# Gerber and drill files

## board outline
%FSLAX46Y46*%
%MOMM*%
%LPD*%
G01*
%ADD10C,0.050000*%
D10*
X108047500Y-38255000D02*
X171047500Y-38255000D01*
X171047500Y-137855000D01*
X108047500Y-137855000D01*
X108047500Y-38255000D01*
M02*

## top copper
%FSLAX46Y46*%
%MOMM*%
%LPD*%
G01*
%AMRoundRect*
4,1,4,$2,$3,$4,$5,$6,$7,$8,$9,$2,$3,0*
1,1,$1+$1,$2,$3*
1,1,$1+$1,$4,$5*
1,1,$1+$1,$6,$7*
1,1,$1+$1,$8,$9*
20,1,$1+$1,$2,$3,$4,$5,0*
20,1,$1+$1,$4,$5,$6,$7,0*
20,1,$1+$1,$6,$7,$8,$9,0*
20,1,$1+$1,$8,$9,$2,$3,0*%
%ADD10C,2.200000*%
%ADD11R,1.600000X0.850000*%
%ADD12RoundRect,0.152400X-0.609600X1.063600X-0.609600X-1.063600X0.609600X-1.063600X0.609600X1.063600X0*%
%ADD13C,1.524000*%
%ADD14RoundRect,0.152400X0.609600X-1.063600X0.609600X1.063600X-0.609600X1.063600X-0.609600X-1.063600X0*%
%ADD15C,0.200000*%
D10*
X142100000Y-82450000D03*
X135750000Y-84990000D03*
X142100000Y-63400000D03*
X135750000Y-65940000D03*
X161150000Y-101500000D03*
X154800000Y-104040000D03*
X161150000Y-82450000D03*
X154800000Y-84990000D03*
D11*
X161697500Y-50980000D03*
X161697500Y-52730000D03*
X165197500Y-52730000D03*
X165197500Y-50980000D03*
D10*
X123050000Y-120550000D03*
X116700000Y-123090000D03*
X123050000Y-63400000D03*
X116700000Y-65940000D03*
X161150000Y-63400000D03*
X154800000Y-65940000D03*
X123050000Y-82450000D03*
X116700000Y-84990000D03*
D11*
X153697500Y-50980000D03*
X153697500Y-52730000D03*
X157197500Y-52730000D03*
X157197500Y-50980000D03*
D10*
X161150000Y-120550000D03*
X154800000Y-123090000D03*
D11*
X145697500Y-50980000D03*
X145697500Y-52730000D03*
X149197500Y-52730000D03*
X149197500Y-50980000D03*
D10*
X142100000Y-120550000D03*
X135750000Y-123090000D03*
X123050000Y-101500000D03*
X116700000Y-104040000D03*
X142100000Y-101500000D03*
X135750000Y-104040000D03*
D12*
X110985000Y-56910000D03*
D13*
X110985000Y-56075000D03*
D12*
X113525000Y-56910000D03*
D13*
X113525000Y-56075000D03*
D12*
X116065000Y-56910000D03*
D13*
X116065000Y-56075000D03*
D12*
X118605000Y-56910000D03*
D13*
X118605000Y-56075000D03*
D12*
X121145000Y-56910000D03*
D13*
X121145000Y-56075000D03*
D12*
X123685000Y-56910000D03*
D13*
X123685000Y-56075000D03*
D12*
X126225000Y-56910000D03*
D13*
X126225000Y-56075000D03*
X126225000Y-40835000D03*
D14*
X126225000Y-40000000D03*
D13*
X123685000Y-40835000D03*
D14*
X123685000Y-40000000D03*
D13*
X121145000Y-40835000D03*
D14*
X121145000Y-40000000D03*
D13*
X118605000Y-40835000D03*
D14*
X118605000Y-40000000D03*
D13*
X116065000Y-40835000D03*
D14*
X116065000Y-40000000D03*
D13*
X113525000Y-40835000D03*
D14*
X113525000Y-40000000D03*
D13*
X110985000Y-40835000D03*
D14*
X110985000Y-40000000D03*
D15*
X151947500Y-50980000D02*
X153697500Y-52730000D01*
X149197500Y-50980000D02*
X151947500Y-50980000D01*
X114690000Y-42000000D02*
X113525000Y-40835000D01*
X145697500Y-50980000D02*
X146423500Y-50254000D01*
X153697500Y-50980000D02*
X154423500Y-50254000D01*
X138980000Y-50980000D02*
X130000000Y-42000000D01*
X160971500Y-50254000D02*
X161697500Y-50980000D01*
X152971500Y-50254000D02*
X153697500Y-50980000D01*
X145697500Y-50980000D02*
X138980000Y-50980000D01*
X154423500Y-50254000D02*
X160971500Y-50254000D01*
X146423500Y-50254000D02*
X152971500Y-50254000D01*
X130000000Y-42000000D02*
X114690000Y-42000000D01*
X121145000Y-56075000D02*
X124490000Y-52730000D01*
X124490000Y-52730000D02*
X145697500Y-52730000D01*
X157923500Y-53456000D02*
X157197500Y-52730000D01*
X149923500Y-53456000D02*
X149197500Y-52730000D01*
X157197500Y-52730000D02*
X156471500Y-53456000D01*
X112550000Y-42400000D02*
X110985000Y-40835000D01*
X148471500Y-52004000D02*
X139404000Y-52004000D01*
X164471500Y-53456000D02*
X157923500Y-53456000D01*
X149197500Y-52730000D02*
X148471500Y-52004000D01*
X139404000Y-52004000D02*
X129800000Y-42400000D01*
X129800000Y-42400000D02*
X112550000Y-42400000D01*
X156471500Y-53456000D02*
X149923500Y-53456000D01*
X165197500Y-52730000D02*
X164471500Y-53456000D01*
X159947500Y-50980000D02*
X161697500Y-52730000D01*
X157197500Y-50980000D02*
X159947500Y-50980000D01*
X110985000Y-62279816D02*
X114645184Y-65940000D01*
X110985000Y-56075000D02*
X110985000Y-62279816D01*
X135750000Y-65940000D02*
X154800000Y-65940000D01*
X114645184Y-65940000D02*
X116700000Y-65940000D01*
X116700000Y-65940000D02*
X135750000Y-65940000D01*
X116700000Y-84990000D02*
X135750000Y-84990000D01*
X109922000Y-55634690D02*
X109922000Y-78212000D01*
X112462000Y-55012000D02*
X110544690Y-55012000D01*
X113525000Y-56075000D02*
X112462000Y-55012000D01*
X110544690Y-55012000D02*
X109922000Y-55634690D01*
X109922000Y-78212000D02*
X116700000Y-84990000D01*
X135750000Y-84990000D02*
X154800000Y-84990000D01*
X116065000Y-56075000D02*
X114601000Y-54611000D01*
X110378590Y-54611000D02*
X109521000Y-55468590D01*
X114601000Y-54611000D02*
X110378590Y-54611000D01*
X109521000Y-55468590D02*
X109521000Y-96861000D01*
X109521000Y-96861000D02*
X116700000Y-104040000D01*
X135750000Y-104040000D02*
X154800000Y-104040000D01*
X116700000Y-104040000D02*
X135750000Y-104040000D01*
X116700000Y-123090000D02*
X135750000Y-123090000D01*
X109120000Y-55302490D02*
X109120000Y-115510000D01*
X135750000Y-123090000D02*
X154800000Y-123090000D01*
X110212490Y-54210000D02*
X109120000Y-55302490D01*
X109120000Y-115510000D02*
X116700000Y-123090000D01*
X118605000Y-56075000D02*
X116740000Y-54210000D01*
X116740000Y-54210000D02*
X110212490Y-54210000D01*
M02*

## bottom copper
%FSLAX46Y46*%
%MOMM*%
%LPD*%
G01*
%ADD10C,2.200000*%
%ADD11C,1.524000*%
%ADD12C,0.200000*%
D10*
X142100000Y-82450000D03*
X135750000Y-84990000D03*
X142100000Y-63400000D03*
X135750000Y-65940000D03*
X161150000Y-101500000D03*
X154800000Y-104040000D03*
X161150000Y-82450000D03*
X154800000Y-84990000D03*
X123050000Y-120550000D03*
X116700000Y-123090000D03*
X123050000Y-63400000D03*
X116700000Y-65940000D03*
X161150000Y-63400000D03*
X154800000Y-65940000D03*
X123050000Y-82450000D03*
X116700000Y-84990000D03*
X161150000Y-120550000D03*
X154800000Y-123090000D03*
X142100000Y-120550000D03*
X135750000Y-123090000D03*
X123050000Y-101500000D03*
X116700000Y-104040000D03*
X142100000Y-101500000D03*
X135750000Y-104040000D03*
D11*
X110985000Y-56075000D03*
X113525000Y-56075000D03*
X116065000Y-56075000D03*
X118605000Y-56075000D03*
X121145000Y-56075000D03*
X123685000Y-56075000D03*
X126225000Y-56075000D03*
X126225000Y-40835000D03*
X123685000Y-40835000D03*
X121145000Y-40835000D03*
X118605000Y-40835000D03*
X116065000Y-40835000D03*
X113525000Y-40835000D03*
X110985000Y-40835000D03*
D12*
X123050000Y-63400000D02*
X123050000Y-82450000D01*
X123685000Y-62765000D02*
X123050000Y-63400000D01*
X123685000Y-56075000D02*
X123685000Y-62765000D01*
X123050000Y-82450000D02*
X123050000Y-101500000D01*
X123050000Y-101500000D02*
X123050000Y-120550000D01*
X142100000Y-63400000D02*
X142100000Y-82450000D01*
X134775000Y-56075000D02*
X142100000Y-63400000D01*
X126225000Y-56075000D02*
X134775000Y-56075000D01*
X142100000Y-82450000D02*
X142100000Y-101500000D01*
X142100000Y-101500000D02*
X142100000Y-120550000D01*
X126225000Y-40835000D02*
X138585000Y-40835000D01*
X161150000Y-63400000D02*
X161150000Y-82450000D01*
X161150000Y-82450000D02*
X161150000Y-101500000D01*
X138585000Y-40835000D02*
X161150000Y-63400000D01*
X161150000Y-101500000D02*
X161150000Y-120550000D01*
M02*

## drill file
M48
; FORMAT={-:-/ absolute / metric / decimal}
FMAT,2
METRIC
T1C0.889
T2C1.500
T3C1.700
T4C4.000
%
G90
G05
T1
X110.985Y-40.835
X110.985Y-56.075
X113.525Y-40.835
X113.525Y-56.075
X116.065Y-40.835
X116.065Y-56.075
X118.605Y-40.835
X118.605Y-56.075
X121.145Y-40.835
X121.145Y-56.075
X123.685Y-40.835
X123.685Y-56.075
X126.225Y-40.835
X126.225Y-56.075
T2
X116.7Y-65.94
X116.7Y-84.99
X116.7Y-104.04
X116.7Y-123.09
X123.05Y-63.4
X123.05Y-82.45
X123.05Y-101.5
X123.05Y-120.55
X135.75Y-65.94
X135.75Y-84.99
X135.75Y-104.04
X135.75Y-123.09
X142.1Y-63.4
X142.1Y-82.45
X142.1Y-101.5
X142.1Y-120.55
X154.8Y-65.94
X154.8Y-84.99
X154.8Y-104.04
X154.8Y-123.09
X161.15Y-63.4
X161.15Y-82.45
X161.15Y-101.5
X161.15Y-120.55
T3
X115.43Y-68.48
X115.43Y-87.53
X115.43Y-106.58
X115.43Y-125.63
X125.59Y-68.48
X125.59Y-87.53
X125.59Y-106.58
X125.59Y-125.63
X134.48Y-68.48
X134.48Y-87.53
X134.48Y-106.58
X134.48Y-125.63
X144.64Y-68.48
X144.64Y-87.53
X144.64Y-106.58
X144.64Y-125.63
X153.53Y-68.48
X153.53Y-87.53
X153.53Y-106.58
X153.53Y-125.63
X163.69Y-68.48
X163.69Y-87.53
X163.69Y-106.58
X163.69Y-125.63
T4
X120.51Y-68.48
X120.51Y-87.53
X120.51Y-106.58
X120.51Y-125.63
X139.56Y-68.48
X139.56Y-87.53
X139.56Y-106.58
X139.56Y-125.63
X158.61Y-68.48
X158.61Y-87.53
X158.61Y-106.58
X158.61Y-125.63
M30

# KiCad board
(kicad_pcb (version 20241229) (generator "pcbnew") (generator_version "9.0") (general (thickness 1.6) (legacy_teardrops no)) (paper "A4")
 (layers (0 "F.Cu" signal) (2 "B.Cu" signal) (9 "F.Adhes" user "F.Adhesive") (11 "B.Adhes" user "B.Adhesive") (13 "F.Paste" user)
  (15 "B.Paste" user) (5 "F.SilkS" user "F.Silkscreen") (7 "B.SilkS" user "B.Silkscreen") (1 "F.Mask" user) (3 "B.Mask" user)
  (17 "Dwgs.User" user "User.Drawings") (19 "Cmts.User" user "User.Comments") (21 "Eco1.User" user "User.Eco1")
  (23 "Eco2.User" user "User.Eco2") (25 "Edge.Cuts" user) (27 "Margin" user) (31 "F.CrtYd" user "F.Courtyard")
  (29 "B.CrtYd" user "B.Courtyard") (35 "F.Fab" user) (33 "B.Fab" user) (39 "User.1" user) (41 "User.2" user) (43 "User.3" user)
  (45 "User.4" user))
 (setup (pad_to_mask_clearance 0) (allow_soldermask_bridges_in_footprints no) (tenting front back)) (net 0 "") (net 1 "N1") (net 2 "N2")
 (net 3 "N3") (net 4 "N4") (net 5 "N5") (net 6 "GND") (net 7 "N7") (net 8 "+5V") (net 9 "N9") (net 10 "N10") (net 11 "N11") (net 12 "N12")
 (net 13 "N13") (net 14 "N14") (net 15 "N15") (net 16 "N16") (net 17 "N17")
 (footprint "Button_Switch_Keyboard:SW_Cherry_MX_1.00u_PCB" (layer "F.Cu") (at 142.1 82.45)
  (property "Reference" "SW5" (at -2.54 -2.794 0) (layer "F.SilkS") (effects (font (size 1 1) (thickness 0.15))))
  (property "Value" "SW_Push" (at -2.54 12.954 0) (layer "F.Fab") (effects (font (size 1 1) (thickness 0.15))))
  (pad "" np_thru_hole circle (at -7.62 5.08) (size 1.7 1.7) (drill 1.7) (layers "*.Cu" "*.Mask"))
  (pad "" np_thru_hole circle (at -2.54 5.08) (size 4 4) (drill 4) (layers "*.Cu" "*.Mask"))
  (pad "" np_thru_hole circle (at 2.54 5.08) (size 1.7 1.7) (drill 1.7) (layers "*.Cu" "*.Mask"))
  (pad "1" thru_hole circle (at 0 0) (size 2.2 2.2) (drill 1.5) (layers "*.Cu" "*.Mask") (remove_unused_layers no) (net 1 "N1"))
  (pad "2" thru_hole circle (at -6.35 2.54) (size 2.2 2.2) (drill 1.5) (layers "*.Cu" "*.Mask") (remove_unused_layers no) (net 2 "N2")))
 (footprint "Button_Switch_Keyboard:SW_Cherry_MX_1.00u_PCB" (layer "F.Cu") (at 142.1 63.4)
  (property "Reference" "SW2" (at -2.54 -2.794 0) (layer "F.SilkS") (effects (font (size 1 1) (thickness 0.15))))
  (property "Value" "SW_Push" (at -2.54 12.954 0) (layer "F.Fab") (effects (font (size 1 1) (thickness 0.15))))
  (pad "" np_thru_hole circle (at -7.62 5.08) (size 1.7 1.7) (drill 1.7) (layers "*.Cu" "*.Mask"))
  (pad "" np_thru_hole circle (at -2.54 5.08) (size 4 4) (drill 4) (layers "*.Cu" "*.Mask"))
  (pad "" np_thru_hole circle (at 2.54 5.08) (size 1.7 1.7) (drill 1.7) (layers "*.Cu" "*.Mask"))
  (pad "1" thru_hole circle (at 0 0) (size 2.2 2.2) (drill 1.5) (layers "*.Cu" "*.Mask") (remove_unused_layers no) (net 1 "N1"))
  (pad "2" thru_hole circle (at -6.35 2.54) (size 2.2 2.2) (drill 1.5) (layers "*.Cu" "*.Mask") (remove_unused_layers no) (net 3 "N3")))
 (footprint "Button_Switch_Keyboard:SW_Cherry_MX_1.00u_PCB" (layer "F.Cu") (at 161.15 101.5)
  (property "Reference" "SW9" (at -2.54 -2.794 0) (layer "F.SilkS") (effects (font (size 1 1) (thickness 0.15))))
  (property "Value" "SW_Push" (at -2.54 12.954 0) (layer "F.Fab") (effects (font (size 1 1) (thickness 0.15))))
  (pad "" np_thru_hole circle (at -7.62 5.08) (size 1.7 1.7) (drill 1.7) (layers "*.Cu" "*.Mask"))
  (pad "" np_thru_hole circle (at -2.54 5.08) (size 4 4) (drill 4) (layers "*.Cu" "*.Mask"))
  (pad "" np_thru_hole circle (at 2.54 5.08) (size 1.7 1.7) (drill 1.7) (layers "*.Cu" "*.Mask"))
  (pad "1" thru_hole circle (at 0 0) (size 2.2 2.2) (drill 1.5) (layers "*.Cu" "*.Mask") (remove_unused_layers no) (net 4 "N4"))
  (pad "2" thru_hole circle (at -6.35 2.54) (size 2.2 2.2) (drill 1.5) (layers "*.Cu" "*.Mask") (remove_unused_layers no) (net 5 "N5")))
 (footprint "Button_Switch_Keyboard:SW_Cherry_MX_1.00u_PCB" (layer "F.Cu") (at 161.15 82.45)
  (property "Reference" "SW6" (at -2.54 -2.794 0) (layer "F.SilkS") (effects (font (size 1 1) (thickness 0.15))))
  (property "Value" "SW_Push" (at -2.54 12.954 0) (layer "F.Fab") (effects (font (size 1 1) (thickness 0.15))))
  (pad "" np_thru_hole circle (at -7.62 5.08) (size 1.7 1.7) (drill 1.7) (layers "*.Cu" "*.Mask"))
  (pad "" np_thru_hole circle (at -2.54 5.08) (size 4 4) (drill 4) (layers "*.Cu" "*.Mask"))
  (pad "" np_thru_hole circle (at 2.54 5.08) (size 1.7 1.7) (drill 1.7) (layers "*.Cu" "*.Mask"))
  (pad "1" thru_hole circle (at 0 0) (size 2.2 2.2) (drill 1.5) (layers "*.Cu" "*.Mask") (remove_unused_layers no) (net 4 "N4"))
  (pad "2" thru_hole circle (at -6.35 2.54) (size 2.2 2.2) (drill 1.5) (layers "*.Cu" "*.Mask") (remove_unused_layers no) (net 2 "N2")))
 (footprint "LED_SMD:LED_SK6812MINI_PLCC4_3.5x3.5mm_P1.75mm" (layer "F.Cu") (at 163.4475 51.855)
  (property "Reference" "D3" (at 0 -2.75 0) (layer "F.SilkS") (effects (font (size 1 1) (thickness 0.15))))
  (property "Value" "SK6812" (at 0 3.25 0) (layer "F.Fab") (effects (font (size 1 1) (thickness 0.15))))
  (pad "1" smd rect (at -1.75 -0.875) (size 1.6 0.85) (layers "F.Cu" "F.Mask" "F.Paste") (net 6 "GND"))
  (pad "2" smd rect (at -1.75 0.875) (size 1.6 0.85) (layers "F.Cu" "F.Mask" "F.Paste") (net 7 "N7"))
  (pad "3" smd rect (at 1.75 0.875) (size 1.6 0.85) (layers "F.Cu" "F.Mask" "F.Paste") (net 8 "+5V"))
  (pad "4" smd rect (at 1.75 -0.875) (size 1.6 0.85) (layers "F.Cu" "F.Mask" "F.Paste") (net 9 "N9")))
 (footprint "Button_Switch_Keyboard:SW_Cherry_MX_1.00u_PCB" (layer "F.Cu") (at 123.05 120.55)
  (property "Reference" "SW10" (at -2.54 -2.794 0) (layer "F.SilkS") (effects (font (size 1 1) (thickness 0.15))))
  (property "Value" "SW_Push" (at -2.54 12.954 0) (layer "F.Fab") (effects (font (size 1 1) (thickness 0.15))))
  (pad "" np_thru_hole circle (at -7.62 5.08) (size 1.7 1.7) (drill 1.7) (layers "*.Cu" "*.Mask"))
  (pad "" np_thru_hole circle (at -2.54 5.08) (size 4 4) (drill 4) (layers "*.Cu" "*.Mask"))
  (pad "" np_thru_hole circle (at 2.54 5.08) (size 1.7 1.7) (drill 1.7) (layers "*.Cu" "*.Mask"))
  (pad "1" thru_hole circle (at 0 0) (size 2.2 2.2) (drill 1.5) (layers "*.Cu" "*.Mask") (remove_unused_layers no) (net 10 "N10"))
  (pad "2" thru_hole circle (at -6.35 2.54) (size 2.2 2.2) (drill 1.5) (layers "*.Cu" "*.Mask") (remove_unused_layers no) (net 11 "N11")))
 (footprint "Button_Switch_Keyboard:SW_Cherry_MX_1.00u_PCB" (layer "F.Cu") (at 123.05 63.4)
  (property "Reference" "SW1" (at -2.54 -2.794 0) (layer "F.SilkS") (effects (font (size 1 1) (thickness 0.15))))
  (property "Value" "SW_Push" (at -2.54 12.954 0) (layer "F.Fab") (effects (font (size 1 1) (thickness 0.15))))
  (pad "" np_thru_hole circle (at -7.62 5.08) (size 1.7 1.7) (drill 1.7) (layers "*.Cu" "*.Mask"))
  (pad "" np_thru_hole circle (at -2.54 5.08) (size 4 4) (drill 4) (layers "*.Cu" "*.Mask"))
  (pad "" np_thru_hole circle (at 2.54 5.08) (size 1.7 1.7) (drill 1.7) (layers "*.Cu" "*.Mask"))
  (pad "1" thru_hole circle (at 0 0) (size 2.2 2.2) (drill 1.5) (layers "*.Cu" "*.Mask") (remove_unused_layers no) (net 10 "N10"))
  (pad "2" thru_hole circle (at -6.35 2.54) (size 2.2 2.2) (drill 1.5) (layers "*.Cu" "*.Mask") (remove_unused_layers no) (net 3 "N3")))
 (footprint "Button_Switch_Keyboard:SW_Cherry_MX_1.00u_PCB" (layer "F.Cu") (at 161.15 63.4)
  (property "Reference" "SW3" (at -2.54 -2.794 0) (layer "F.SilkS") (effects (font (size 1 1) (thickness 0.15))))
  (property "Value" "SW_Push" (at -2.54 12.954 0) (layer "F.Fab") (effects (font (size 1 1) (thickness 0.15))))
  (pad "" np_thru_hole circle (at -7.62 5.08) (size 1.7 1.7) (drill 1.7) (layers "*.Cu" "*.Mask"))
  (pad "" np_thru_hole circle (at -2.54 5.08) (size 4 4) (drill 4) (layers "*.Cu" "*.Mask"))
  (pad "" np_thru_hole circle (at 2.54 5.08) (size 1.7 1.7) (drill 1.7) (layers "*.Cu" "*.Mask"))
  (pad "1" thru_hole circle (at 0 0) (size 2.2 2.2) (drill 1.5) (layers "*.Cu" "*.Mask") (remove_unused_layers no) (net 4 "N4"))
  (pad "2" thru_hole circle (at -6.35 2.54) (size 2.2 2.2) (drill 1.5) (layers "*.Cu" "*.Mask") (remove_unused_layers no) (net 3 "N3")))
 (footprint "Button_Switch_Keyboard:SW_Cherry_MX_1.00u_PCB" (layer "F.Cu") (at 123.05 82.45)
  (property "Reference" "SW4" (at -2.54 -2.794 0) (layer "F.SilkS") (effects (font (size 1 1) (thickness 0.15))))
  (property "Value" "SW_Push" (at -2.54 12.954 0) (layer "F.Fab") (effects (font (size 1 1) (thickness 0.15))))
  (pad "" np_thru_hole circle (at -7.62 5.08) (size 1.7 1.7) (drill 1.7) (layers "*.Cu" "*.Mask"))
  (pad "" np_thru_hole circle (at -2.54 5.08) (size 4 4) (drill 4) (layers "*.Cu" "*.Mask"))
  (pad "" np_thru_hole circle (at 2.54 5.08) (size 1.7 1.7) (drill 1.7) (layers "*.Cu" "*.Mask"))
  (pad "1" thru_hole circle (at 0 0) (size 2.2 2.2) (drill 1.5) (layers "*.Cu" "*.Mask") (remove_unused_layers no) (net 10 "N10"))
  (pad "2" thru_hole circle (at -6.35 2.54) (size 2.2 2.2) (drill 1.5) (layers "*.Cu" "*.Mask") (remove_unused_layers no) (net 2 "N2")))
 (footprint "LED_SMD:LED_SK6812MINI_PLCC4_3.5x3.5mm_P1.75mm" (layer "F.Cu") (at 155.4475 51.855)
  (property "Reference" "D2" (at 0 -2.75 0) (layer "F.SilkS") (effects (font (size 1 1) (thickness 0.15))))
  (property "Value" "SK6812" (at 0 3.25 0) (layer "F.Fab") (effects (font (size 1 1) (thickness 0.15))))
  (pad "1" smd rect (at -1.75 -0.875) (size 1.6 0.85) (layers "F.Cu" "F.Mask" "F.Paste") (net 6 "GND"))
  (pad "2" smd rect (at -1.75 0.875) (size 1.6 0.85) (layers "F.Cu" "F.Mask" "F.Paste") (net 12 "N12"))
  (pad "3" smd rect (at 1.75 0.875) (size 1.6 0.85) (layers "F.Cu" "F.Mask" "F.Paste") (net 8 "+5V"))
  (pad "4" smd rect (at 1.75 -0.875) (size 1.6 0.85) (layers "F.Cu" "F.Mask" "F.Paste") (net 7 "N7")))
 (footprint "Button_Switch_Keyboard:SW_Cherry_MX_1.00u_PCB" (layer "F.Cu") (at 161.15 120.55)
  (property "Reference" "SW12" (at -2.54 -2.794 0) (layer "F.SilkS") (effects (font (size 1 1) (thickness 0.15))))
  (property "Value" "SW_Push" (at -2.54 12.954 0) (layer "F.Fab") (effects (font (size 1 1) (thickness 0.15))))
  (pad "" np_thru_hole circle (at -7.62 5.08) (size 1.7 1.7) (drill 1.7) (layers "*.Cu" "*.Mask"))
  (pad "" np_thru_hole circle (at -2.54 5.08) (size 4 4) (drill 4) (layers "*.Cu" "*.Mask"))
  (pad "" np_thru_hole circle (at 2.54 5.08) (size 1.7 1.7) (drill 1.7) (layers "*.Cu" "*.Mask"))
  (pad "1" thru_hole circle (at 0 0) (size 2.2 2.2) (drill 1.5) (layers "*.Cu" "*.Mask") (remove_unused_layers no) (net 4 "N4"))
  (pad "2" thru_hole circle (at -6.35 2.54) (size 2.2 2.2) (drill 1.5) (layers "*.Cu" "*.Mask") (remove_unused_layers no) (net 11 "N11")))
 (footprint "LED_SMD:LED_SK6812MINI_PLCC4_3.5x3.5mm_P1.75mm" (layer "F.Cu") (at 147.4475 51.855)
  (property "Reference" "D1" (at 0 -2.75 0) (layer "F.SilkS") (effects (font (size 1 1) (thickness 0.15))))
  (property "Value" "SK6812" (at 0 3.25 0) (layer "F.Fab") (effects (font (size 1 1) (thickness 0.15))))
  (pad "1" smd rect (at -1.75 -0.875) (size 1.6 0.85) (layers "F.Cu" "F.Mask" "F.Paste") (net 6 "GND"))
  (pad "2" smd rect (at -1.75 0.875) (size 1.6 0.85) (layers "F.Cu" "F.Mask" "F.Paste") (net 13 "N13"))
  (pad "3" smd rect (at 1.75 0.875) (size 1.6 0.85) (layers "F.Cu" "F.Mask" "F.Paste") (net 8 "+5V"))
  (pad "4" smd rect (at 1.75 -0.875) (size 1.6 0.85) (layers "F.Cu" "F.Mask" "F.Paste") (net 12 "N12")))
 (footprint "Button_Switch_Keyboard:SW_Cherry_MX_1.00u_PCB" (layer "F.Cu") (at 142.1 120.55)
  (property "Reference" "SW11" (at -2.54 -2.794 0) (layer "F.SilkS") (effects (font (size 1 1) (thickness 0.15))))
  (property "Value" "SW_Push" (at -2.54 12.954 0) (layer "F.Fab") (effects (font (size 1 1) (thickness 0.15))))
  (pad "" np_thru_hole circle (at -7.62 5.08) (size 1.7 1.7) (drill 1.7) (layers "*.Cu" "*.Mask"))
  (pad "" np_thru_hole circle (at -2.54 5.08) (size 4 4) (drill 4) (layers "*.Cu" "*.Mask"))
  (pad "" np_thru_hole circle (at 2.54 5.08) (size 1.7 1.7) (drill 1.7) (layers "*.Cu" "*.Mask"))
  (pad "1" thru_hole circle (at 0 0) (size 2.2 2.2) (drill 1.5) (layers "*.Cu" "*.Mask") (remove_unused_layers no) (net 1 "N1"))
  (pad "2" thru_hole circle (at -6.35 2.54) (size 2.2 2.2) (drill 1.5) (layers "*.Cu" "*.Mask") (remove_unused_layers no) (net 11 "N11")))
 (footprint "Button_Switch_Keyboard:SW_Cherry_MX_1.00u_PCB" (layer "F.Cu") (at 123.05 101.5)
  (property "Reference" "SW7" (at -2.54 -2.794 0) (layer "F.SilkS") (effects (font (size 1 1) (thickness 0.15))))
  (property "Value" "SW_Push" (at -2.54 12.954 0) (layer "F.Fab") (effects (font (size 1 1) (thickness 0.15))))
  (pad "" np_thru_hole circle (at -7.62 5.08) (size 1.7 1.7) (drill 1.7) (layers "*.Cu" "*.Mask"))
  (pad "" np_thru_hole circle (at -2.54 5.08) (size 4 4) (drill 4) (layers "*.Cu" "*.Mask"))
  (pad "" np_thru_hole circle (at 2.54 5.08) (size 1.7 1.7) (drill 1.7) (layers "*.Cu" "*.Mask"))
  (pad "1" thru_hole circle (at 0 0) (size 2.2 2.2) (drill 1.5) (layers "*.Cu" "*.Mask") (remove_unused_layers no) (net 10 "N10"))
  (pad "2" thru_hole circle (at -6.35 2.54) (size 2.2 2.2) (drill 1.5) (layers "*.Cu" "*.Mask") (remove_unused_layers no) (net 5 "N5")))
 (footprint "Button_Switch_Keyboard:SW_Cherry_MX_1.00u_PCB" (layer "F.Cu") (at 142.1 101.5)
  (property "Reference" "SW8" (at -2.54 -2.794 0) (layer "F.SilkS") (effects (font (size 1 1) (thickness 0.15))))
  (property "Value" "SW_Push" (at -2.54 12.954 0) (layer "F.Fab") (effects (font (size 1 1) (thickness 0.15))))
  (pad "" np_thru_hole circle (at -7.62 5.08) (size 1.7 1.7) (drill 1.7) (layers "*.Cu" "*.Mask"))
  (pad "" np_thru_hole circle (at -2.54 5.08) (size 4 4) (drill 4) (layers "*.Cu" "*.Mask"))
  (pad "" np_thru_hole circle (at 2.54 5.08) (size 1.7 1.7) (drill 1.7) (layers "*.Cu" "*.Mask"))
  (pad "1" thru_hole circle (at 0 0) (size 2.2 2.2) (drill 1.5) (layers "*.Cu" "*.Mask") (remove_unused_layers no) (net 1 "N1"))
  (pad "2" thru_hole circle (at -6.35 2.54) (size 2.2 2.2) (drill 1.5) (layers "*.Cu" "*.Mask") (remove_unused_layers no) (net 5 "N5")))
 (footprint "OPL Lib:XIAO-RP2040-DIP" (layer "F.Cu") (at 118.605 48.455 90)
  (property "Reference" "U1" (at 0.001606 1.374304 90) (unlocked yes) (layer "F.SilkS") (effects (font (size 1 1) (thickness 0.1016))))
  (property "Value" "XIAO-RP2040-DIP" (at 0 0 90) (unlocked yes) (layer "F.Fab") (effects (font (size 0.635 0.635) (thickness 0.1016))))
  (pad "1" smd roundrect (at -8.455 -7.62 270) (size 2.432 1.524) (layers "F.Cu" "F.Mask") (roundrect_rratio 0.1) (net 3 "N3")
   (thermal_bridge_angle 45))
  (pad "1" thru_hole circle (at -7.62 -7.62 270) (size 1.524 1.524) (drill 0.889) (layers "*.Cu" "*.Mask") (remove_unused_layers no)
   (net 3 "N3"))
  (pad "2" smd roundrect (at -8.455 -5.08 270) (size 2.432 1.524) (layers "F.Cu" "F.Mask") (roundrect_rratio 0.1) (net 2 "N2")
   (thermal_bridge_angle 45))
  (pad "2" thru_hole circle (at -7.62 -5.08 270) (size 1.524 1.524) (drill 0.889) (layers "*.Cu" "*.Mask") (remove_unused_layers no)
   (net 2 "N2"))
  (pad "3" smd roundrect (at -8.455 -2.54 270) (size 2.432 1.524) (layers "F.Cu" "F.Mask") (roundrect_rratio 0.1) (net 5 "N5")
   (thermal_bridge_angle 45))
  (pad "3" thru_hole circle (at -7.62 -2.54 270) (size 1.524 1.524) (drill 0.889) (layers "*.Cu" "*.Mask") (remove_unused_layers no)
   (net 5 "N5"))
  (pad "4" smd roundrect (at -8.455 0 270) (size 2.432 1.524) (layers "F.Cu" "F.Mask") (roundrect_rratio 0.1) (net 11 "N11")
   (thermal_bridge_angle 45))
  (pad "4" thru_hole circle (at -7.62 0 270) (size 1.524 1.524) (drill 0.889) (layers "*.Cu" "*.Mask") (remove_unused_layers no)
   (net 11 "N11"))
  (pad "5" smd roundrect (at -8.455 2.54 270) (size 2.432 1.524) (layers "F.Cu" "F.Mask") (roundrect_rratio 0.1) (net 13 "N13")
   (thermal_bridge_angle 45))
  (pad "5" thru_hole circle (at -7.62 2.54 270) (size 1.524 1.524) (drill 0.889) (layers "*.Cu" "*.Mask") (remove_unused_layers no)
   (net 13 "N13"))
  (pad "6" smd roundrect (at -8.455 5.08 270) (size 2.432 1.524) (layers "F.Cu" "F.Mask") (roundrect_rratio 0.1) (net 10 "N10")
   (thermal_bridge_angle 45))
  (pad "6" thru_hole circle (at -7.62 5.08 270) (size 1.524 1.524) (drill 0.889) (layers "*.Cu" "*.Mask") (remove_unused_layers no)
   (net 10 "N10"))
  (pad "7" smd roundrect (at -8.455 7.62 270) (size 2.432 1.524) (layers "F.Cu" "F.Mask") (roundrect_rratio 0.1) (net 1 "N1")
   (thermal_bridge_angle 45))
  (pad "7" thru_hole circle (at -7.62 7.62 270) (size 1.524 1.524) (drill 0.889) (layers "*.Cu" "*.Mask") (remove_unused_layers no)
   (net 1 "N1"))
  (pad "8" thru_hole circle (at 7.62 7.62 90) (size 1.524 1.524) (drill 0.889) (layers "*.Cu" "*.Mask") (remove_unused_layers no)
   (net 4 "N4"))
  (pad "8" smd roundrect (at 8.455 7.62 90) (size 2.432 1.524) (layers "F.Cu" "F.Mask") (roundrect_rratio 0.1) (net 4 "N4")
   (thermal_bridge_angle 45))
  (pad "9" thru_hole circle (at 7.62 5.08 90) (size 1.524 1.524) (drill 0.889) (layers "*.Cu" "*.Mask") (remove_unused_layers no)
   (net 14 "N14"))
  (pad "9" smd roundrect (at 8.455 5.08 90) (size 2.432 1.524) (layers "F.Cu" "F.Mask") (roundrect_rratio 0.1) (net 14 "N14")
   (thermal_bridge_angle 45))
  (pad "10" thru_hole circle (at 7.62 2.54 90) (size 1.524 1.524) (drill 0.889) (layers "*.Cu" "*.Mask") (remove_unused_layers no)
   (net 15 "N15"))
  (pad "10" smd roundrect (at 8.455 2.54 90) (size 2.432 1.524) (layers "F.Cu" "F.Mask") (roundrect_rratio 0.1) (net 15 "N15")
   (thermal_bridge_angle 45))
  (pad "11" thru_hole circle (at 7.62 0 90) (size 1.524 1.524) (drill 0.889) (layers "*.Cu" "*.Mask") (remove_unused_layers no)
   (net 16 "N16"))
  (pad "11" smd roundrect (at 8.455 0 90) (size 2.432 1.524) (layers "F.Cu" "F.Mask") (roundrect_rratio 0.1) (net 16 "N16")
   (thermal_bridge_angle 45))
  (pad "12" thru_hole circle (at 7.62 -2.54 90) (size 1.524 1.524) (drill 0.889) (layers "*.Cu" "*.Mask") (remove_unused_layers no)
   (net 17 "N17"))
  (pad "12" smd roundrect (at 8.455 -2.54 90) (size 2.432 1.524) (layers "F.Cu" "F.Mask") (roundrect_rratio 0.1) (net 17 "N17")
   (thermal_bridge_angle 45))
  (pad "13" thru_hole circle (at 7.62 -5.08 90) (size 1.524 1.524) (drill 0.889) (layers "*.Cu" "*.Mask") (remove_unused_layers no)
   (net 6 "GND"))
  (pad "13" smd roundrect (at 8.455 -5.08 90) (size 2.432 1.524) (layers "F.Cu" "F.Mask") (roundrect_rratio 0.1) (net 6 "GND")
   (thermal_bridge_angle 45))
  (pad "14" thru_hole circle (at 7.62 -7.62 90) (size 1.524 1.524) (drill 0.889) (layers "*.Cu" "*.Mask") (remove_unused_layers no)
   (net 8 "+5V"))
  (pad "14" smd roundrect (at 8.455 -7.62 90) (size 2.432 1.524) (layers "F.Cu" "F.Mask") (roundrect_rratio 0.1) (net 8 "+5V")
   (thermal_bridge_angle 45)))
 (gr_rect (start 108.0475 38.255) (end 171.0475 137.855) (stroke (width 0.05) (type default)) (fill no) (layer "Edge.Cuts"))
 (segment (start 151.9475 50.98) (end 153.6975 52.73) (width 0.2) (layer "F.Cu") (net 12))
 (segment (start 149.1975 50.98) (end 151.9475 50.98) (width 0.2) (layer "F.Cu") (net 12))
 (segment (start 114.69 42) (end 113.525 40.835) (width 0.2) (layer "F.Cu") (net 6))
 (segment (start 145.6975 50.98) (end 146.4235 50.254) (width 0.2) (layer "F.Cu") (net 6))
 (segment (start 153.6975 50.98) (end 154.4235 50.254) (width 0.2) (layer "F.Cu") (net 6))
 (segment (start 138.98 50.98) (end 130 42) (width 0.2) (layer "F.Cu") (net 6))
 (segment (start 160.9715 50.254) (end 161.6975 50.98) (width 0.2) (layer "F.Cu") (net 6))
 (segment (start 152.9715 50.254) (end 153.6975 50.98) (width 0.2) (layer "F.Cu") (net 6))
 (segment (start 145.6975 50.98) (end 138.98 50.98) (width 0.2) (layer "F.Cu") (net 6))
 (segment (start 154.4235 50.254) (end 160.9715 50.254) (width 0.2) (layer "F.Cu") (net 6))
 (segment (start 146.4235 50.254) (end 152.9715 50.254) (width 0.2) (layer "F.Cu") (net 6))
 (segment (start 130 42) (end 114.69 42) (width 0.2) (layer "F.Cu") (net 6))
 (segment (start 121.145 56.075) (end 124.49 52.73) (width 0.2) (layer "F.Cu") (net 13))
 (segment (start 124.49 52.73) (end 145.6975 52.73) (width 0.2) (layer "F.Cu") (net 13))
 (segment (start 157.9235 53.456) (end 157.1975 52.73) (width 0.2) (layer "F.Cu") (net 8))
 (segment (start 149.9235 53.456) (end 149.1975 52.73) (width 0.2) (layer "F.Cu") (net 8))
 (segment (start 157.1975 52.73) (end 156.4715 53.456) (width 0.2) (layer "F.Cu") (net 8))
 (segment (start 112.55 42.4) (end 110.985 40.835) (width 0.2) (layer "F.Cu") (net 8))
 (segment (start 148.4715 52.004) (end 139.404 52.004) (width 0.2) (layer "F.Cu") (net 8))
 (segment (start 164.4715 53.456) (end 157.9235 53.456) (width 0.2) (layer "F.Cu") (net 8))
 (segment (start 149.1975 52.73) (end 148.4715 52.004) (width 0.2) (layer "F.Cu") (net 8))
 (segment (start 139.404 52.004) (end 129.8 42.4) (width 0.2) (layer "F.Cu") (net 8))
 (segment (start 129.8 42.4) (end 112.55 42.4) (width 0.2) (layer "F.Cu") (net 8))
 (segment (start 156.4715 53.456) (end 149.9235 53.456) (width 0.2) (layer "F.Cu") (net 8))
 (segment (start 165.1975 52.73) (end 164.4715 53.456) (width 0.2) (layer "F.Cu") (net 8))
 (segment (start 159.9475 50.98) (end 161.6975 52.73) (width 0.2) (layer "F.Cu") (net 7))
 (segment (start 157.1975 50.98) (end 159.9475 50.98) (width 0.2) (layer "F.Cu") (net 7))
 (segment (start 110.985 62.279816) (end 114.645184 65.94) (width 0.2) (layer "F.Cu") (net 3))
 (segment (start 110.985 56.075) (end 110.985 62.279816) (width 0.2) (layer "F.Cu") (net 3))
 (segment (start 135.75 65.94) (end 154.8 65.94) (width 0.2) (layer "F.Cu") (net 3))
 (segment (start 114.645184 65.94) (end 116.7 65.94) (width 0.2) (layer "F.Cu") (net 3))
 (segment (start 116.7 65.94) (end 135.75 65.94) (width 0.2) (layer "F.Cu") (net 3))
 (segment (start 123.05 63.4) (end 123.05 82.45) (width 0.2) (layer "B.Cu") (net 10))
 (segment (start 123.685 62.765) (end 123.05 63.4) (width 0.2) (layer "B.Cu") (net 10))
 (segment (start 123.685 56.075) (end 123.685 62.765) (width 0.2) (layer "B.Cu") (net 10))
 (segment (start 123.05 82.45) (end 123.05 101.5) (width 0.2) (layer "B.Cu") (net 10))
 (segment (start 123.05 101.5) (end 123.05 120.55) (width 0.2) (layer "B.Cu") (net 10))
 (segment (start 142.1 63.4) (end 142.1 82.45) (width 0.2) (layer "B.Cu") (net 1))
 (segment (start 134.775 56.075) (end 142.1 63.4) (width 0.2) (layer "B.Cu") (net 1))
 (segment (start 126.225 56.075) (end 134.775 56.075) (width 0.2) (layer "B.Cu") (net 1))
 (segment (start 142.1 82.45) (end 142.1 101.5) (width 0.2) (layer "B.Cu") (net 1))
 (segment (start 142.1 101.5) (end 142.1 120.55) (width 0.2) (layer "B.Cu") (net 1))
 (segment (start 126.225 40.835) (end 138.585 40.835) (width 0.2) (layer "B.Cu") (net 4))
 (segment (start 161.15 63.4) (end 161.15 82.45) (width 0.2) (layer "B.Cu") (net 4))
 (segment (start 161.15 82.45) (end 161.15 101.5) (width 0.2) (layer "B.Cu") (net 4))
 (segment (start 138.585 40.835) (end 161.15 63.4) (width 0.2) (layer "B.Cu") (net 4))
 (segment (start 161.15 101.5) (end 161.15 120.55) (width 0.2) (layer "B.Cu") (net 4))
 (segment (start 116.7 84.99) (end 135.75 84.99) (width 0.2) (layer "F.Cu") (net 2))
 (segment (start 109.922 55.63469) (end 109.922 78.212) (width 0.2) (layer "F.Cu") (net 2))
 (segment (start 112.462 55.012) (end 110.54469 55.012) (width 0.2) (layer "F.Cu") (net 2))
 (segment (start 113.525 56.075) (end 112.462 55.012) (width 0.2) (layer "F.Cu") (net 2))
 (segment (start 110.54469 55.012) (end 109.922 55.63469) (width 0.2) (layer "F.Cu") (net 2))
 (segment (start 109.922 78.212) (end 116.7 84.99) (width 0.2) (layer "F.Cu") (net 2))
 (segment (start 135.75 84.99) (end 154.8 84.99) (width 0.2) (layer "F.Cu") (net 2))
 (segment (start 116.065 56.075) (end 114.601 54.611) (width 0.2) (layer "F.Cu") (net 5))
 (segment (start 110.37859 54.611) (end 109.521 55.46859) (width 0.2) (layer "F.Cu") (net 5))
 (segment (start 114.601 54.611) (end 110.37859 54.611) (width 0.2) (layer "F.Cu") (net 5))
 (segment (start 109.521 55.46859) (end 109.521 96.861) (width 0.2) (layer "F.Cu") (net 5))
 (segment (start 109.521 96.861) (end 116.7 104.04) (width 0.2) (layer "F.Cu") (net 5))
 (segment (start 135.75 104.04) (end 154.8 104.04) (width 0.2) (layer "F.Cu") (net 5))
 (segment (start 116.7 104.04) (end 135.75 104.04) (width 0.2) (layer "F.Cu") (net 5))
 (segment (start 116.7 123.09) (end 135.75 123.09) (width 0.2) (layer "F.Cu") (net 11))
 (segment (start 109.12 55.30249) (end 109.12 115.51) (width 0.2) (layer "F.Cu") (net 11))
 (segment (start 135.75 123.09) (end 154.8 123.09) (width 0.2) (layer "F.Cu") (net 11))
 (segment (start 110.21249 54.21) (end 109.12 55.30249) (width 0.2) (layer "F.Cu") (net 11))
 (segment (start 109.12 115.51) (end 116.7 123.09) (width 0.2) (layer "F.Cu") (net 11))
 (segment (start 118.605 56.075) (end 116.74 54.21) (width 0.2) (layer "F.Cu") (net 11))
 (segment (start 116.74 54.21) (end 110.21249 54.21) (width 0.2) (layer "F.Cu") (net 11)))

